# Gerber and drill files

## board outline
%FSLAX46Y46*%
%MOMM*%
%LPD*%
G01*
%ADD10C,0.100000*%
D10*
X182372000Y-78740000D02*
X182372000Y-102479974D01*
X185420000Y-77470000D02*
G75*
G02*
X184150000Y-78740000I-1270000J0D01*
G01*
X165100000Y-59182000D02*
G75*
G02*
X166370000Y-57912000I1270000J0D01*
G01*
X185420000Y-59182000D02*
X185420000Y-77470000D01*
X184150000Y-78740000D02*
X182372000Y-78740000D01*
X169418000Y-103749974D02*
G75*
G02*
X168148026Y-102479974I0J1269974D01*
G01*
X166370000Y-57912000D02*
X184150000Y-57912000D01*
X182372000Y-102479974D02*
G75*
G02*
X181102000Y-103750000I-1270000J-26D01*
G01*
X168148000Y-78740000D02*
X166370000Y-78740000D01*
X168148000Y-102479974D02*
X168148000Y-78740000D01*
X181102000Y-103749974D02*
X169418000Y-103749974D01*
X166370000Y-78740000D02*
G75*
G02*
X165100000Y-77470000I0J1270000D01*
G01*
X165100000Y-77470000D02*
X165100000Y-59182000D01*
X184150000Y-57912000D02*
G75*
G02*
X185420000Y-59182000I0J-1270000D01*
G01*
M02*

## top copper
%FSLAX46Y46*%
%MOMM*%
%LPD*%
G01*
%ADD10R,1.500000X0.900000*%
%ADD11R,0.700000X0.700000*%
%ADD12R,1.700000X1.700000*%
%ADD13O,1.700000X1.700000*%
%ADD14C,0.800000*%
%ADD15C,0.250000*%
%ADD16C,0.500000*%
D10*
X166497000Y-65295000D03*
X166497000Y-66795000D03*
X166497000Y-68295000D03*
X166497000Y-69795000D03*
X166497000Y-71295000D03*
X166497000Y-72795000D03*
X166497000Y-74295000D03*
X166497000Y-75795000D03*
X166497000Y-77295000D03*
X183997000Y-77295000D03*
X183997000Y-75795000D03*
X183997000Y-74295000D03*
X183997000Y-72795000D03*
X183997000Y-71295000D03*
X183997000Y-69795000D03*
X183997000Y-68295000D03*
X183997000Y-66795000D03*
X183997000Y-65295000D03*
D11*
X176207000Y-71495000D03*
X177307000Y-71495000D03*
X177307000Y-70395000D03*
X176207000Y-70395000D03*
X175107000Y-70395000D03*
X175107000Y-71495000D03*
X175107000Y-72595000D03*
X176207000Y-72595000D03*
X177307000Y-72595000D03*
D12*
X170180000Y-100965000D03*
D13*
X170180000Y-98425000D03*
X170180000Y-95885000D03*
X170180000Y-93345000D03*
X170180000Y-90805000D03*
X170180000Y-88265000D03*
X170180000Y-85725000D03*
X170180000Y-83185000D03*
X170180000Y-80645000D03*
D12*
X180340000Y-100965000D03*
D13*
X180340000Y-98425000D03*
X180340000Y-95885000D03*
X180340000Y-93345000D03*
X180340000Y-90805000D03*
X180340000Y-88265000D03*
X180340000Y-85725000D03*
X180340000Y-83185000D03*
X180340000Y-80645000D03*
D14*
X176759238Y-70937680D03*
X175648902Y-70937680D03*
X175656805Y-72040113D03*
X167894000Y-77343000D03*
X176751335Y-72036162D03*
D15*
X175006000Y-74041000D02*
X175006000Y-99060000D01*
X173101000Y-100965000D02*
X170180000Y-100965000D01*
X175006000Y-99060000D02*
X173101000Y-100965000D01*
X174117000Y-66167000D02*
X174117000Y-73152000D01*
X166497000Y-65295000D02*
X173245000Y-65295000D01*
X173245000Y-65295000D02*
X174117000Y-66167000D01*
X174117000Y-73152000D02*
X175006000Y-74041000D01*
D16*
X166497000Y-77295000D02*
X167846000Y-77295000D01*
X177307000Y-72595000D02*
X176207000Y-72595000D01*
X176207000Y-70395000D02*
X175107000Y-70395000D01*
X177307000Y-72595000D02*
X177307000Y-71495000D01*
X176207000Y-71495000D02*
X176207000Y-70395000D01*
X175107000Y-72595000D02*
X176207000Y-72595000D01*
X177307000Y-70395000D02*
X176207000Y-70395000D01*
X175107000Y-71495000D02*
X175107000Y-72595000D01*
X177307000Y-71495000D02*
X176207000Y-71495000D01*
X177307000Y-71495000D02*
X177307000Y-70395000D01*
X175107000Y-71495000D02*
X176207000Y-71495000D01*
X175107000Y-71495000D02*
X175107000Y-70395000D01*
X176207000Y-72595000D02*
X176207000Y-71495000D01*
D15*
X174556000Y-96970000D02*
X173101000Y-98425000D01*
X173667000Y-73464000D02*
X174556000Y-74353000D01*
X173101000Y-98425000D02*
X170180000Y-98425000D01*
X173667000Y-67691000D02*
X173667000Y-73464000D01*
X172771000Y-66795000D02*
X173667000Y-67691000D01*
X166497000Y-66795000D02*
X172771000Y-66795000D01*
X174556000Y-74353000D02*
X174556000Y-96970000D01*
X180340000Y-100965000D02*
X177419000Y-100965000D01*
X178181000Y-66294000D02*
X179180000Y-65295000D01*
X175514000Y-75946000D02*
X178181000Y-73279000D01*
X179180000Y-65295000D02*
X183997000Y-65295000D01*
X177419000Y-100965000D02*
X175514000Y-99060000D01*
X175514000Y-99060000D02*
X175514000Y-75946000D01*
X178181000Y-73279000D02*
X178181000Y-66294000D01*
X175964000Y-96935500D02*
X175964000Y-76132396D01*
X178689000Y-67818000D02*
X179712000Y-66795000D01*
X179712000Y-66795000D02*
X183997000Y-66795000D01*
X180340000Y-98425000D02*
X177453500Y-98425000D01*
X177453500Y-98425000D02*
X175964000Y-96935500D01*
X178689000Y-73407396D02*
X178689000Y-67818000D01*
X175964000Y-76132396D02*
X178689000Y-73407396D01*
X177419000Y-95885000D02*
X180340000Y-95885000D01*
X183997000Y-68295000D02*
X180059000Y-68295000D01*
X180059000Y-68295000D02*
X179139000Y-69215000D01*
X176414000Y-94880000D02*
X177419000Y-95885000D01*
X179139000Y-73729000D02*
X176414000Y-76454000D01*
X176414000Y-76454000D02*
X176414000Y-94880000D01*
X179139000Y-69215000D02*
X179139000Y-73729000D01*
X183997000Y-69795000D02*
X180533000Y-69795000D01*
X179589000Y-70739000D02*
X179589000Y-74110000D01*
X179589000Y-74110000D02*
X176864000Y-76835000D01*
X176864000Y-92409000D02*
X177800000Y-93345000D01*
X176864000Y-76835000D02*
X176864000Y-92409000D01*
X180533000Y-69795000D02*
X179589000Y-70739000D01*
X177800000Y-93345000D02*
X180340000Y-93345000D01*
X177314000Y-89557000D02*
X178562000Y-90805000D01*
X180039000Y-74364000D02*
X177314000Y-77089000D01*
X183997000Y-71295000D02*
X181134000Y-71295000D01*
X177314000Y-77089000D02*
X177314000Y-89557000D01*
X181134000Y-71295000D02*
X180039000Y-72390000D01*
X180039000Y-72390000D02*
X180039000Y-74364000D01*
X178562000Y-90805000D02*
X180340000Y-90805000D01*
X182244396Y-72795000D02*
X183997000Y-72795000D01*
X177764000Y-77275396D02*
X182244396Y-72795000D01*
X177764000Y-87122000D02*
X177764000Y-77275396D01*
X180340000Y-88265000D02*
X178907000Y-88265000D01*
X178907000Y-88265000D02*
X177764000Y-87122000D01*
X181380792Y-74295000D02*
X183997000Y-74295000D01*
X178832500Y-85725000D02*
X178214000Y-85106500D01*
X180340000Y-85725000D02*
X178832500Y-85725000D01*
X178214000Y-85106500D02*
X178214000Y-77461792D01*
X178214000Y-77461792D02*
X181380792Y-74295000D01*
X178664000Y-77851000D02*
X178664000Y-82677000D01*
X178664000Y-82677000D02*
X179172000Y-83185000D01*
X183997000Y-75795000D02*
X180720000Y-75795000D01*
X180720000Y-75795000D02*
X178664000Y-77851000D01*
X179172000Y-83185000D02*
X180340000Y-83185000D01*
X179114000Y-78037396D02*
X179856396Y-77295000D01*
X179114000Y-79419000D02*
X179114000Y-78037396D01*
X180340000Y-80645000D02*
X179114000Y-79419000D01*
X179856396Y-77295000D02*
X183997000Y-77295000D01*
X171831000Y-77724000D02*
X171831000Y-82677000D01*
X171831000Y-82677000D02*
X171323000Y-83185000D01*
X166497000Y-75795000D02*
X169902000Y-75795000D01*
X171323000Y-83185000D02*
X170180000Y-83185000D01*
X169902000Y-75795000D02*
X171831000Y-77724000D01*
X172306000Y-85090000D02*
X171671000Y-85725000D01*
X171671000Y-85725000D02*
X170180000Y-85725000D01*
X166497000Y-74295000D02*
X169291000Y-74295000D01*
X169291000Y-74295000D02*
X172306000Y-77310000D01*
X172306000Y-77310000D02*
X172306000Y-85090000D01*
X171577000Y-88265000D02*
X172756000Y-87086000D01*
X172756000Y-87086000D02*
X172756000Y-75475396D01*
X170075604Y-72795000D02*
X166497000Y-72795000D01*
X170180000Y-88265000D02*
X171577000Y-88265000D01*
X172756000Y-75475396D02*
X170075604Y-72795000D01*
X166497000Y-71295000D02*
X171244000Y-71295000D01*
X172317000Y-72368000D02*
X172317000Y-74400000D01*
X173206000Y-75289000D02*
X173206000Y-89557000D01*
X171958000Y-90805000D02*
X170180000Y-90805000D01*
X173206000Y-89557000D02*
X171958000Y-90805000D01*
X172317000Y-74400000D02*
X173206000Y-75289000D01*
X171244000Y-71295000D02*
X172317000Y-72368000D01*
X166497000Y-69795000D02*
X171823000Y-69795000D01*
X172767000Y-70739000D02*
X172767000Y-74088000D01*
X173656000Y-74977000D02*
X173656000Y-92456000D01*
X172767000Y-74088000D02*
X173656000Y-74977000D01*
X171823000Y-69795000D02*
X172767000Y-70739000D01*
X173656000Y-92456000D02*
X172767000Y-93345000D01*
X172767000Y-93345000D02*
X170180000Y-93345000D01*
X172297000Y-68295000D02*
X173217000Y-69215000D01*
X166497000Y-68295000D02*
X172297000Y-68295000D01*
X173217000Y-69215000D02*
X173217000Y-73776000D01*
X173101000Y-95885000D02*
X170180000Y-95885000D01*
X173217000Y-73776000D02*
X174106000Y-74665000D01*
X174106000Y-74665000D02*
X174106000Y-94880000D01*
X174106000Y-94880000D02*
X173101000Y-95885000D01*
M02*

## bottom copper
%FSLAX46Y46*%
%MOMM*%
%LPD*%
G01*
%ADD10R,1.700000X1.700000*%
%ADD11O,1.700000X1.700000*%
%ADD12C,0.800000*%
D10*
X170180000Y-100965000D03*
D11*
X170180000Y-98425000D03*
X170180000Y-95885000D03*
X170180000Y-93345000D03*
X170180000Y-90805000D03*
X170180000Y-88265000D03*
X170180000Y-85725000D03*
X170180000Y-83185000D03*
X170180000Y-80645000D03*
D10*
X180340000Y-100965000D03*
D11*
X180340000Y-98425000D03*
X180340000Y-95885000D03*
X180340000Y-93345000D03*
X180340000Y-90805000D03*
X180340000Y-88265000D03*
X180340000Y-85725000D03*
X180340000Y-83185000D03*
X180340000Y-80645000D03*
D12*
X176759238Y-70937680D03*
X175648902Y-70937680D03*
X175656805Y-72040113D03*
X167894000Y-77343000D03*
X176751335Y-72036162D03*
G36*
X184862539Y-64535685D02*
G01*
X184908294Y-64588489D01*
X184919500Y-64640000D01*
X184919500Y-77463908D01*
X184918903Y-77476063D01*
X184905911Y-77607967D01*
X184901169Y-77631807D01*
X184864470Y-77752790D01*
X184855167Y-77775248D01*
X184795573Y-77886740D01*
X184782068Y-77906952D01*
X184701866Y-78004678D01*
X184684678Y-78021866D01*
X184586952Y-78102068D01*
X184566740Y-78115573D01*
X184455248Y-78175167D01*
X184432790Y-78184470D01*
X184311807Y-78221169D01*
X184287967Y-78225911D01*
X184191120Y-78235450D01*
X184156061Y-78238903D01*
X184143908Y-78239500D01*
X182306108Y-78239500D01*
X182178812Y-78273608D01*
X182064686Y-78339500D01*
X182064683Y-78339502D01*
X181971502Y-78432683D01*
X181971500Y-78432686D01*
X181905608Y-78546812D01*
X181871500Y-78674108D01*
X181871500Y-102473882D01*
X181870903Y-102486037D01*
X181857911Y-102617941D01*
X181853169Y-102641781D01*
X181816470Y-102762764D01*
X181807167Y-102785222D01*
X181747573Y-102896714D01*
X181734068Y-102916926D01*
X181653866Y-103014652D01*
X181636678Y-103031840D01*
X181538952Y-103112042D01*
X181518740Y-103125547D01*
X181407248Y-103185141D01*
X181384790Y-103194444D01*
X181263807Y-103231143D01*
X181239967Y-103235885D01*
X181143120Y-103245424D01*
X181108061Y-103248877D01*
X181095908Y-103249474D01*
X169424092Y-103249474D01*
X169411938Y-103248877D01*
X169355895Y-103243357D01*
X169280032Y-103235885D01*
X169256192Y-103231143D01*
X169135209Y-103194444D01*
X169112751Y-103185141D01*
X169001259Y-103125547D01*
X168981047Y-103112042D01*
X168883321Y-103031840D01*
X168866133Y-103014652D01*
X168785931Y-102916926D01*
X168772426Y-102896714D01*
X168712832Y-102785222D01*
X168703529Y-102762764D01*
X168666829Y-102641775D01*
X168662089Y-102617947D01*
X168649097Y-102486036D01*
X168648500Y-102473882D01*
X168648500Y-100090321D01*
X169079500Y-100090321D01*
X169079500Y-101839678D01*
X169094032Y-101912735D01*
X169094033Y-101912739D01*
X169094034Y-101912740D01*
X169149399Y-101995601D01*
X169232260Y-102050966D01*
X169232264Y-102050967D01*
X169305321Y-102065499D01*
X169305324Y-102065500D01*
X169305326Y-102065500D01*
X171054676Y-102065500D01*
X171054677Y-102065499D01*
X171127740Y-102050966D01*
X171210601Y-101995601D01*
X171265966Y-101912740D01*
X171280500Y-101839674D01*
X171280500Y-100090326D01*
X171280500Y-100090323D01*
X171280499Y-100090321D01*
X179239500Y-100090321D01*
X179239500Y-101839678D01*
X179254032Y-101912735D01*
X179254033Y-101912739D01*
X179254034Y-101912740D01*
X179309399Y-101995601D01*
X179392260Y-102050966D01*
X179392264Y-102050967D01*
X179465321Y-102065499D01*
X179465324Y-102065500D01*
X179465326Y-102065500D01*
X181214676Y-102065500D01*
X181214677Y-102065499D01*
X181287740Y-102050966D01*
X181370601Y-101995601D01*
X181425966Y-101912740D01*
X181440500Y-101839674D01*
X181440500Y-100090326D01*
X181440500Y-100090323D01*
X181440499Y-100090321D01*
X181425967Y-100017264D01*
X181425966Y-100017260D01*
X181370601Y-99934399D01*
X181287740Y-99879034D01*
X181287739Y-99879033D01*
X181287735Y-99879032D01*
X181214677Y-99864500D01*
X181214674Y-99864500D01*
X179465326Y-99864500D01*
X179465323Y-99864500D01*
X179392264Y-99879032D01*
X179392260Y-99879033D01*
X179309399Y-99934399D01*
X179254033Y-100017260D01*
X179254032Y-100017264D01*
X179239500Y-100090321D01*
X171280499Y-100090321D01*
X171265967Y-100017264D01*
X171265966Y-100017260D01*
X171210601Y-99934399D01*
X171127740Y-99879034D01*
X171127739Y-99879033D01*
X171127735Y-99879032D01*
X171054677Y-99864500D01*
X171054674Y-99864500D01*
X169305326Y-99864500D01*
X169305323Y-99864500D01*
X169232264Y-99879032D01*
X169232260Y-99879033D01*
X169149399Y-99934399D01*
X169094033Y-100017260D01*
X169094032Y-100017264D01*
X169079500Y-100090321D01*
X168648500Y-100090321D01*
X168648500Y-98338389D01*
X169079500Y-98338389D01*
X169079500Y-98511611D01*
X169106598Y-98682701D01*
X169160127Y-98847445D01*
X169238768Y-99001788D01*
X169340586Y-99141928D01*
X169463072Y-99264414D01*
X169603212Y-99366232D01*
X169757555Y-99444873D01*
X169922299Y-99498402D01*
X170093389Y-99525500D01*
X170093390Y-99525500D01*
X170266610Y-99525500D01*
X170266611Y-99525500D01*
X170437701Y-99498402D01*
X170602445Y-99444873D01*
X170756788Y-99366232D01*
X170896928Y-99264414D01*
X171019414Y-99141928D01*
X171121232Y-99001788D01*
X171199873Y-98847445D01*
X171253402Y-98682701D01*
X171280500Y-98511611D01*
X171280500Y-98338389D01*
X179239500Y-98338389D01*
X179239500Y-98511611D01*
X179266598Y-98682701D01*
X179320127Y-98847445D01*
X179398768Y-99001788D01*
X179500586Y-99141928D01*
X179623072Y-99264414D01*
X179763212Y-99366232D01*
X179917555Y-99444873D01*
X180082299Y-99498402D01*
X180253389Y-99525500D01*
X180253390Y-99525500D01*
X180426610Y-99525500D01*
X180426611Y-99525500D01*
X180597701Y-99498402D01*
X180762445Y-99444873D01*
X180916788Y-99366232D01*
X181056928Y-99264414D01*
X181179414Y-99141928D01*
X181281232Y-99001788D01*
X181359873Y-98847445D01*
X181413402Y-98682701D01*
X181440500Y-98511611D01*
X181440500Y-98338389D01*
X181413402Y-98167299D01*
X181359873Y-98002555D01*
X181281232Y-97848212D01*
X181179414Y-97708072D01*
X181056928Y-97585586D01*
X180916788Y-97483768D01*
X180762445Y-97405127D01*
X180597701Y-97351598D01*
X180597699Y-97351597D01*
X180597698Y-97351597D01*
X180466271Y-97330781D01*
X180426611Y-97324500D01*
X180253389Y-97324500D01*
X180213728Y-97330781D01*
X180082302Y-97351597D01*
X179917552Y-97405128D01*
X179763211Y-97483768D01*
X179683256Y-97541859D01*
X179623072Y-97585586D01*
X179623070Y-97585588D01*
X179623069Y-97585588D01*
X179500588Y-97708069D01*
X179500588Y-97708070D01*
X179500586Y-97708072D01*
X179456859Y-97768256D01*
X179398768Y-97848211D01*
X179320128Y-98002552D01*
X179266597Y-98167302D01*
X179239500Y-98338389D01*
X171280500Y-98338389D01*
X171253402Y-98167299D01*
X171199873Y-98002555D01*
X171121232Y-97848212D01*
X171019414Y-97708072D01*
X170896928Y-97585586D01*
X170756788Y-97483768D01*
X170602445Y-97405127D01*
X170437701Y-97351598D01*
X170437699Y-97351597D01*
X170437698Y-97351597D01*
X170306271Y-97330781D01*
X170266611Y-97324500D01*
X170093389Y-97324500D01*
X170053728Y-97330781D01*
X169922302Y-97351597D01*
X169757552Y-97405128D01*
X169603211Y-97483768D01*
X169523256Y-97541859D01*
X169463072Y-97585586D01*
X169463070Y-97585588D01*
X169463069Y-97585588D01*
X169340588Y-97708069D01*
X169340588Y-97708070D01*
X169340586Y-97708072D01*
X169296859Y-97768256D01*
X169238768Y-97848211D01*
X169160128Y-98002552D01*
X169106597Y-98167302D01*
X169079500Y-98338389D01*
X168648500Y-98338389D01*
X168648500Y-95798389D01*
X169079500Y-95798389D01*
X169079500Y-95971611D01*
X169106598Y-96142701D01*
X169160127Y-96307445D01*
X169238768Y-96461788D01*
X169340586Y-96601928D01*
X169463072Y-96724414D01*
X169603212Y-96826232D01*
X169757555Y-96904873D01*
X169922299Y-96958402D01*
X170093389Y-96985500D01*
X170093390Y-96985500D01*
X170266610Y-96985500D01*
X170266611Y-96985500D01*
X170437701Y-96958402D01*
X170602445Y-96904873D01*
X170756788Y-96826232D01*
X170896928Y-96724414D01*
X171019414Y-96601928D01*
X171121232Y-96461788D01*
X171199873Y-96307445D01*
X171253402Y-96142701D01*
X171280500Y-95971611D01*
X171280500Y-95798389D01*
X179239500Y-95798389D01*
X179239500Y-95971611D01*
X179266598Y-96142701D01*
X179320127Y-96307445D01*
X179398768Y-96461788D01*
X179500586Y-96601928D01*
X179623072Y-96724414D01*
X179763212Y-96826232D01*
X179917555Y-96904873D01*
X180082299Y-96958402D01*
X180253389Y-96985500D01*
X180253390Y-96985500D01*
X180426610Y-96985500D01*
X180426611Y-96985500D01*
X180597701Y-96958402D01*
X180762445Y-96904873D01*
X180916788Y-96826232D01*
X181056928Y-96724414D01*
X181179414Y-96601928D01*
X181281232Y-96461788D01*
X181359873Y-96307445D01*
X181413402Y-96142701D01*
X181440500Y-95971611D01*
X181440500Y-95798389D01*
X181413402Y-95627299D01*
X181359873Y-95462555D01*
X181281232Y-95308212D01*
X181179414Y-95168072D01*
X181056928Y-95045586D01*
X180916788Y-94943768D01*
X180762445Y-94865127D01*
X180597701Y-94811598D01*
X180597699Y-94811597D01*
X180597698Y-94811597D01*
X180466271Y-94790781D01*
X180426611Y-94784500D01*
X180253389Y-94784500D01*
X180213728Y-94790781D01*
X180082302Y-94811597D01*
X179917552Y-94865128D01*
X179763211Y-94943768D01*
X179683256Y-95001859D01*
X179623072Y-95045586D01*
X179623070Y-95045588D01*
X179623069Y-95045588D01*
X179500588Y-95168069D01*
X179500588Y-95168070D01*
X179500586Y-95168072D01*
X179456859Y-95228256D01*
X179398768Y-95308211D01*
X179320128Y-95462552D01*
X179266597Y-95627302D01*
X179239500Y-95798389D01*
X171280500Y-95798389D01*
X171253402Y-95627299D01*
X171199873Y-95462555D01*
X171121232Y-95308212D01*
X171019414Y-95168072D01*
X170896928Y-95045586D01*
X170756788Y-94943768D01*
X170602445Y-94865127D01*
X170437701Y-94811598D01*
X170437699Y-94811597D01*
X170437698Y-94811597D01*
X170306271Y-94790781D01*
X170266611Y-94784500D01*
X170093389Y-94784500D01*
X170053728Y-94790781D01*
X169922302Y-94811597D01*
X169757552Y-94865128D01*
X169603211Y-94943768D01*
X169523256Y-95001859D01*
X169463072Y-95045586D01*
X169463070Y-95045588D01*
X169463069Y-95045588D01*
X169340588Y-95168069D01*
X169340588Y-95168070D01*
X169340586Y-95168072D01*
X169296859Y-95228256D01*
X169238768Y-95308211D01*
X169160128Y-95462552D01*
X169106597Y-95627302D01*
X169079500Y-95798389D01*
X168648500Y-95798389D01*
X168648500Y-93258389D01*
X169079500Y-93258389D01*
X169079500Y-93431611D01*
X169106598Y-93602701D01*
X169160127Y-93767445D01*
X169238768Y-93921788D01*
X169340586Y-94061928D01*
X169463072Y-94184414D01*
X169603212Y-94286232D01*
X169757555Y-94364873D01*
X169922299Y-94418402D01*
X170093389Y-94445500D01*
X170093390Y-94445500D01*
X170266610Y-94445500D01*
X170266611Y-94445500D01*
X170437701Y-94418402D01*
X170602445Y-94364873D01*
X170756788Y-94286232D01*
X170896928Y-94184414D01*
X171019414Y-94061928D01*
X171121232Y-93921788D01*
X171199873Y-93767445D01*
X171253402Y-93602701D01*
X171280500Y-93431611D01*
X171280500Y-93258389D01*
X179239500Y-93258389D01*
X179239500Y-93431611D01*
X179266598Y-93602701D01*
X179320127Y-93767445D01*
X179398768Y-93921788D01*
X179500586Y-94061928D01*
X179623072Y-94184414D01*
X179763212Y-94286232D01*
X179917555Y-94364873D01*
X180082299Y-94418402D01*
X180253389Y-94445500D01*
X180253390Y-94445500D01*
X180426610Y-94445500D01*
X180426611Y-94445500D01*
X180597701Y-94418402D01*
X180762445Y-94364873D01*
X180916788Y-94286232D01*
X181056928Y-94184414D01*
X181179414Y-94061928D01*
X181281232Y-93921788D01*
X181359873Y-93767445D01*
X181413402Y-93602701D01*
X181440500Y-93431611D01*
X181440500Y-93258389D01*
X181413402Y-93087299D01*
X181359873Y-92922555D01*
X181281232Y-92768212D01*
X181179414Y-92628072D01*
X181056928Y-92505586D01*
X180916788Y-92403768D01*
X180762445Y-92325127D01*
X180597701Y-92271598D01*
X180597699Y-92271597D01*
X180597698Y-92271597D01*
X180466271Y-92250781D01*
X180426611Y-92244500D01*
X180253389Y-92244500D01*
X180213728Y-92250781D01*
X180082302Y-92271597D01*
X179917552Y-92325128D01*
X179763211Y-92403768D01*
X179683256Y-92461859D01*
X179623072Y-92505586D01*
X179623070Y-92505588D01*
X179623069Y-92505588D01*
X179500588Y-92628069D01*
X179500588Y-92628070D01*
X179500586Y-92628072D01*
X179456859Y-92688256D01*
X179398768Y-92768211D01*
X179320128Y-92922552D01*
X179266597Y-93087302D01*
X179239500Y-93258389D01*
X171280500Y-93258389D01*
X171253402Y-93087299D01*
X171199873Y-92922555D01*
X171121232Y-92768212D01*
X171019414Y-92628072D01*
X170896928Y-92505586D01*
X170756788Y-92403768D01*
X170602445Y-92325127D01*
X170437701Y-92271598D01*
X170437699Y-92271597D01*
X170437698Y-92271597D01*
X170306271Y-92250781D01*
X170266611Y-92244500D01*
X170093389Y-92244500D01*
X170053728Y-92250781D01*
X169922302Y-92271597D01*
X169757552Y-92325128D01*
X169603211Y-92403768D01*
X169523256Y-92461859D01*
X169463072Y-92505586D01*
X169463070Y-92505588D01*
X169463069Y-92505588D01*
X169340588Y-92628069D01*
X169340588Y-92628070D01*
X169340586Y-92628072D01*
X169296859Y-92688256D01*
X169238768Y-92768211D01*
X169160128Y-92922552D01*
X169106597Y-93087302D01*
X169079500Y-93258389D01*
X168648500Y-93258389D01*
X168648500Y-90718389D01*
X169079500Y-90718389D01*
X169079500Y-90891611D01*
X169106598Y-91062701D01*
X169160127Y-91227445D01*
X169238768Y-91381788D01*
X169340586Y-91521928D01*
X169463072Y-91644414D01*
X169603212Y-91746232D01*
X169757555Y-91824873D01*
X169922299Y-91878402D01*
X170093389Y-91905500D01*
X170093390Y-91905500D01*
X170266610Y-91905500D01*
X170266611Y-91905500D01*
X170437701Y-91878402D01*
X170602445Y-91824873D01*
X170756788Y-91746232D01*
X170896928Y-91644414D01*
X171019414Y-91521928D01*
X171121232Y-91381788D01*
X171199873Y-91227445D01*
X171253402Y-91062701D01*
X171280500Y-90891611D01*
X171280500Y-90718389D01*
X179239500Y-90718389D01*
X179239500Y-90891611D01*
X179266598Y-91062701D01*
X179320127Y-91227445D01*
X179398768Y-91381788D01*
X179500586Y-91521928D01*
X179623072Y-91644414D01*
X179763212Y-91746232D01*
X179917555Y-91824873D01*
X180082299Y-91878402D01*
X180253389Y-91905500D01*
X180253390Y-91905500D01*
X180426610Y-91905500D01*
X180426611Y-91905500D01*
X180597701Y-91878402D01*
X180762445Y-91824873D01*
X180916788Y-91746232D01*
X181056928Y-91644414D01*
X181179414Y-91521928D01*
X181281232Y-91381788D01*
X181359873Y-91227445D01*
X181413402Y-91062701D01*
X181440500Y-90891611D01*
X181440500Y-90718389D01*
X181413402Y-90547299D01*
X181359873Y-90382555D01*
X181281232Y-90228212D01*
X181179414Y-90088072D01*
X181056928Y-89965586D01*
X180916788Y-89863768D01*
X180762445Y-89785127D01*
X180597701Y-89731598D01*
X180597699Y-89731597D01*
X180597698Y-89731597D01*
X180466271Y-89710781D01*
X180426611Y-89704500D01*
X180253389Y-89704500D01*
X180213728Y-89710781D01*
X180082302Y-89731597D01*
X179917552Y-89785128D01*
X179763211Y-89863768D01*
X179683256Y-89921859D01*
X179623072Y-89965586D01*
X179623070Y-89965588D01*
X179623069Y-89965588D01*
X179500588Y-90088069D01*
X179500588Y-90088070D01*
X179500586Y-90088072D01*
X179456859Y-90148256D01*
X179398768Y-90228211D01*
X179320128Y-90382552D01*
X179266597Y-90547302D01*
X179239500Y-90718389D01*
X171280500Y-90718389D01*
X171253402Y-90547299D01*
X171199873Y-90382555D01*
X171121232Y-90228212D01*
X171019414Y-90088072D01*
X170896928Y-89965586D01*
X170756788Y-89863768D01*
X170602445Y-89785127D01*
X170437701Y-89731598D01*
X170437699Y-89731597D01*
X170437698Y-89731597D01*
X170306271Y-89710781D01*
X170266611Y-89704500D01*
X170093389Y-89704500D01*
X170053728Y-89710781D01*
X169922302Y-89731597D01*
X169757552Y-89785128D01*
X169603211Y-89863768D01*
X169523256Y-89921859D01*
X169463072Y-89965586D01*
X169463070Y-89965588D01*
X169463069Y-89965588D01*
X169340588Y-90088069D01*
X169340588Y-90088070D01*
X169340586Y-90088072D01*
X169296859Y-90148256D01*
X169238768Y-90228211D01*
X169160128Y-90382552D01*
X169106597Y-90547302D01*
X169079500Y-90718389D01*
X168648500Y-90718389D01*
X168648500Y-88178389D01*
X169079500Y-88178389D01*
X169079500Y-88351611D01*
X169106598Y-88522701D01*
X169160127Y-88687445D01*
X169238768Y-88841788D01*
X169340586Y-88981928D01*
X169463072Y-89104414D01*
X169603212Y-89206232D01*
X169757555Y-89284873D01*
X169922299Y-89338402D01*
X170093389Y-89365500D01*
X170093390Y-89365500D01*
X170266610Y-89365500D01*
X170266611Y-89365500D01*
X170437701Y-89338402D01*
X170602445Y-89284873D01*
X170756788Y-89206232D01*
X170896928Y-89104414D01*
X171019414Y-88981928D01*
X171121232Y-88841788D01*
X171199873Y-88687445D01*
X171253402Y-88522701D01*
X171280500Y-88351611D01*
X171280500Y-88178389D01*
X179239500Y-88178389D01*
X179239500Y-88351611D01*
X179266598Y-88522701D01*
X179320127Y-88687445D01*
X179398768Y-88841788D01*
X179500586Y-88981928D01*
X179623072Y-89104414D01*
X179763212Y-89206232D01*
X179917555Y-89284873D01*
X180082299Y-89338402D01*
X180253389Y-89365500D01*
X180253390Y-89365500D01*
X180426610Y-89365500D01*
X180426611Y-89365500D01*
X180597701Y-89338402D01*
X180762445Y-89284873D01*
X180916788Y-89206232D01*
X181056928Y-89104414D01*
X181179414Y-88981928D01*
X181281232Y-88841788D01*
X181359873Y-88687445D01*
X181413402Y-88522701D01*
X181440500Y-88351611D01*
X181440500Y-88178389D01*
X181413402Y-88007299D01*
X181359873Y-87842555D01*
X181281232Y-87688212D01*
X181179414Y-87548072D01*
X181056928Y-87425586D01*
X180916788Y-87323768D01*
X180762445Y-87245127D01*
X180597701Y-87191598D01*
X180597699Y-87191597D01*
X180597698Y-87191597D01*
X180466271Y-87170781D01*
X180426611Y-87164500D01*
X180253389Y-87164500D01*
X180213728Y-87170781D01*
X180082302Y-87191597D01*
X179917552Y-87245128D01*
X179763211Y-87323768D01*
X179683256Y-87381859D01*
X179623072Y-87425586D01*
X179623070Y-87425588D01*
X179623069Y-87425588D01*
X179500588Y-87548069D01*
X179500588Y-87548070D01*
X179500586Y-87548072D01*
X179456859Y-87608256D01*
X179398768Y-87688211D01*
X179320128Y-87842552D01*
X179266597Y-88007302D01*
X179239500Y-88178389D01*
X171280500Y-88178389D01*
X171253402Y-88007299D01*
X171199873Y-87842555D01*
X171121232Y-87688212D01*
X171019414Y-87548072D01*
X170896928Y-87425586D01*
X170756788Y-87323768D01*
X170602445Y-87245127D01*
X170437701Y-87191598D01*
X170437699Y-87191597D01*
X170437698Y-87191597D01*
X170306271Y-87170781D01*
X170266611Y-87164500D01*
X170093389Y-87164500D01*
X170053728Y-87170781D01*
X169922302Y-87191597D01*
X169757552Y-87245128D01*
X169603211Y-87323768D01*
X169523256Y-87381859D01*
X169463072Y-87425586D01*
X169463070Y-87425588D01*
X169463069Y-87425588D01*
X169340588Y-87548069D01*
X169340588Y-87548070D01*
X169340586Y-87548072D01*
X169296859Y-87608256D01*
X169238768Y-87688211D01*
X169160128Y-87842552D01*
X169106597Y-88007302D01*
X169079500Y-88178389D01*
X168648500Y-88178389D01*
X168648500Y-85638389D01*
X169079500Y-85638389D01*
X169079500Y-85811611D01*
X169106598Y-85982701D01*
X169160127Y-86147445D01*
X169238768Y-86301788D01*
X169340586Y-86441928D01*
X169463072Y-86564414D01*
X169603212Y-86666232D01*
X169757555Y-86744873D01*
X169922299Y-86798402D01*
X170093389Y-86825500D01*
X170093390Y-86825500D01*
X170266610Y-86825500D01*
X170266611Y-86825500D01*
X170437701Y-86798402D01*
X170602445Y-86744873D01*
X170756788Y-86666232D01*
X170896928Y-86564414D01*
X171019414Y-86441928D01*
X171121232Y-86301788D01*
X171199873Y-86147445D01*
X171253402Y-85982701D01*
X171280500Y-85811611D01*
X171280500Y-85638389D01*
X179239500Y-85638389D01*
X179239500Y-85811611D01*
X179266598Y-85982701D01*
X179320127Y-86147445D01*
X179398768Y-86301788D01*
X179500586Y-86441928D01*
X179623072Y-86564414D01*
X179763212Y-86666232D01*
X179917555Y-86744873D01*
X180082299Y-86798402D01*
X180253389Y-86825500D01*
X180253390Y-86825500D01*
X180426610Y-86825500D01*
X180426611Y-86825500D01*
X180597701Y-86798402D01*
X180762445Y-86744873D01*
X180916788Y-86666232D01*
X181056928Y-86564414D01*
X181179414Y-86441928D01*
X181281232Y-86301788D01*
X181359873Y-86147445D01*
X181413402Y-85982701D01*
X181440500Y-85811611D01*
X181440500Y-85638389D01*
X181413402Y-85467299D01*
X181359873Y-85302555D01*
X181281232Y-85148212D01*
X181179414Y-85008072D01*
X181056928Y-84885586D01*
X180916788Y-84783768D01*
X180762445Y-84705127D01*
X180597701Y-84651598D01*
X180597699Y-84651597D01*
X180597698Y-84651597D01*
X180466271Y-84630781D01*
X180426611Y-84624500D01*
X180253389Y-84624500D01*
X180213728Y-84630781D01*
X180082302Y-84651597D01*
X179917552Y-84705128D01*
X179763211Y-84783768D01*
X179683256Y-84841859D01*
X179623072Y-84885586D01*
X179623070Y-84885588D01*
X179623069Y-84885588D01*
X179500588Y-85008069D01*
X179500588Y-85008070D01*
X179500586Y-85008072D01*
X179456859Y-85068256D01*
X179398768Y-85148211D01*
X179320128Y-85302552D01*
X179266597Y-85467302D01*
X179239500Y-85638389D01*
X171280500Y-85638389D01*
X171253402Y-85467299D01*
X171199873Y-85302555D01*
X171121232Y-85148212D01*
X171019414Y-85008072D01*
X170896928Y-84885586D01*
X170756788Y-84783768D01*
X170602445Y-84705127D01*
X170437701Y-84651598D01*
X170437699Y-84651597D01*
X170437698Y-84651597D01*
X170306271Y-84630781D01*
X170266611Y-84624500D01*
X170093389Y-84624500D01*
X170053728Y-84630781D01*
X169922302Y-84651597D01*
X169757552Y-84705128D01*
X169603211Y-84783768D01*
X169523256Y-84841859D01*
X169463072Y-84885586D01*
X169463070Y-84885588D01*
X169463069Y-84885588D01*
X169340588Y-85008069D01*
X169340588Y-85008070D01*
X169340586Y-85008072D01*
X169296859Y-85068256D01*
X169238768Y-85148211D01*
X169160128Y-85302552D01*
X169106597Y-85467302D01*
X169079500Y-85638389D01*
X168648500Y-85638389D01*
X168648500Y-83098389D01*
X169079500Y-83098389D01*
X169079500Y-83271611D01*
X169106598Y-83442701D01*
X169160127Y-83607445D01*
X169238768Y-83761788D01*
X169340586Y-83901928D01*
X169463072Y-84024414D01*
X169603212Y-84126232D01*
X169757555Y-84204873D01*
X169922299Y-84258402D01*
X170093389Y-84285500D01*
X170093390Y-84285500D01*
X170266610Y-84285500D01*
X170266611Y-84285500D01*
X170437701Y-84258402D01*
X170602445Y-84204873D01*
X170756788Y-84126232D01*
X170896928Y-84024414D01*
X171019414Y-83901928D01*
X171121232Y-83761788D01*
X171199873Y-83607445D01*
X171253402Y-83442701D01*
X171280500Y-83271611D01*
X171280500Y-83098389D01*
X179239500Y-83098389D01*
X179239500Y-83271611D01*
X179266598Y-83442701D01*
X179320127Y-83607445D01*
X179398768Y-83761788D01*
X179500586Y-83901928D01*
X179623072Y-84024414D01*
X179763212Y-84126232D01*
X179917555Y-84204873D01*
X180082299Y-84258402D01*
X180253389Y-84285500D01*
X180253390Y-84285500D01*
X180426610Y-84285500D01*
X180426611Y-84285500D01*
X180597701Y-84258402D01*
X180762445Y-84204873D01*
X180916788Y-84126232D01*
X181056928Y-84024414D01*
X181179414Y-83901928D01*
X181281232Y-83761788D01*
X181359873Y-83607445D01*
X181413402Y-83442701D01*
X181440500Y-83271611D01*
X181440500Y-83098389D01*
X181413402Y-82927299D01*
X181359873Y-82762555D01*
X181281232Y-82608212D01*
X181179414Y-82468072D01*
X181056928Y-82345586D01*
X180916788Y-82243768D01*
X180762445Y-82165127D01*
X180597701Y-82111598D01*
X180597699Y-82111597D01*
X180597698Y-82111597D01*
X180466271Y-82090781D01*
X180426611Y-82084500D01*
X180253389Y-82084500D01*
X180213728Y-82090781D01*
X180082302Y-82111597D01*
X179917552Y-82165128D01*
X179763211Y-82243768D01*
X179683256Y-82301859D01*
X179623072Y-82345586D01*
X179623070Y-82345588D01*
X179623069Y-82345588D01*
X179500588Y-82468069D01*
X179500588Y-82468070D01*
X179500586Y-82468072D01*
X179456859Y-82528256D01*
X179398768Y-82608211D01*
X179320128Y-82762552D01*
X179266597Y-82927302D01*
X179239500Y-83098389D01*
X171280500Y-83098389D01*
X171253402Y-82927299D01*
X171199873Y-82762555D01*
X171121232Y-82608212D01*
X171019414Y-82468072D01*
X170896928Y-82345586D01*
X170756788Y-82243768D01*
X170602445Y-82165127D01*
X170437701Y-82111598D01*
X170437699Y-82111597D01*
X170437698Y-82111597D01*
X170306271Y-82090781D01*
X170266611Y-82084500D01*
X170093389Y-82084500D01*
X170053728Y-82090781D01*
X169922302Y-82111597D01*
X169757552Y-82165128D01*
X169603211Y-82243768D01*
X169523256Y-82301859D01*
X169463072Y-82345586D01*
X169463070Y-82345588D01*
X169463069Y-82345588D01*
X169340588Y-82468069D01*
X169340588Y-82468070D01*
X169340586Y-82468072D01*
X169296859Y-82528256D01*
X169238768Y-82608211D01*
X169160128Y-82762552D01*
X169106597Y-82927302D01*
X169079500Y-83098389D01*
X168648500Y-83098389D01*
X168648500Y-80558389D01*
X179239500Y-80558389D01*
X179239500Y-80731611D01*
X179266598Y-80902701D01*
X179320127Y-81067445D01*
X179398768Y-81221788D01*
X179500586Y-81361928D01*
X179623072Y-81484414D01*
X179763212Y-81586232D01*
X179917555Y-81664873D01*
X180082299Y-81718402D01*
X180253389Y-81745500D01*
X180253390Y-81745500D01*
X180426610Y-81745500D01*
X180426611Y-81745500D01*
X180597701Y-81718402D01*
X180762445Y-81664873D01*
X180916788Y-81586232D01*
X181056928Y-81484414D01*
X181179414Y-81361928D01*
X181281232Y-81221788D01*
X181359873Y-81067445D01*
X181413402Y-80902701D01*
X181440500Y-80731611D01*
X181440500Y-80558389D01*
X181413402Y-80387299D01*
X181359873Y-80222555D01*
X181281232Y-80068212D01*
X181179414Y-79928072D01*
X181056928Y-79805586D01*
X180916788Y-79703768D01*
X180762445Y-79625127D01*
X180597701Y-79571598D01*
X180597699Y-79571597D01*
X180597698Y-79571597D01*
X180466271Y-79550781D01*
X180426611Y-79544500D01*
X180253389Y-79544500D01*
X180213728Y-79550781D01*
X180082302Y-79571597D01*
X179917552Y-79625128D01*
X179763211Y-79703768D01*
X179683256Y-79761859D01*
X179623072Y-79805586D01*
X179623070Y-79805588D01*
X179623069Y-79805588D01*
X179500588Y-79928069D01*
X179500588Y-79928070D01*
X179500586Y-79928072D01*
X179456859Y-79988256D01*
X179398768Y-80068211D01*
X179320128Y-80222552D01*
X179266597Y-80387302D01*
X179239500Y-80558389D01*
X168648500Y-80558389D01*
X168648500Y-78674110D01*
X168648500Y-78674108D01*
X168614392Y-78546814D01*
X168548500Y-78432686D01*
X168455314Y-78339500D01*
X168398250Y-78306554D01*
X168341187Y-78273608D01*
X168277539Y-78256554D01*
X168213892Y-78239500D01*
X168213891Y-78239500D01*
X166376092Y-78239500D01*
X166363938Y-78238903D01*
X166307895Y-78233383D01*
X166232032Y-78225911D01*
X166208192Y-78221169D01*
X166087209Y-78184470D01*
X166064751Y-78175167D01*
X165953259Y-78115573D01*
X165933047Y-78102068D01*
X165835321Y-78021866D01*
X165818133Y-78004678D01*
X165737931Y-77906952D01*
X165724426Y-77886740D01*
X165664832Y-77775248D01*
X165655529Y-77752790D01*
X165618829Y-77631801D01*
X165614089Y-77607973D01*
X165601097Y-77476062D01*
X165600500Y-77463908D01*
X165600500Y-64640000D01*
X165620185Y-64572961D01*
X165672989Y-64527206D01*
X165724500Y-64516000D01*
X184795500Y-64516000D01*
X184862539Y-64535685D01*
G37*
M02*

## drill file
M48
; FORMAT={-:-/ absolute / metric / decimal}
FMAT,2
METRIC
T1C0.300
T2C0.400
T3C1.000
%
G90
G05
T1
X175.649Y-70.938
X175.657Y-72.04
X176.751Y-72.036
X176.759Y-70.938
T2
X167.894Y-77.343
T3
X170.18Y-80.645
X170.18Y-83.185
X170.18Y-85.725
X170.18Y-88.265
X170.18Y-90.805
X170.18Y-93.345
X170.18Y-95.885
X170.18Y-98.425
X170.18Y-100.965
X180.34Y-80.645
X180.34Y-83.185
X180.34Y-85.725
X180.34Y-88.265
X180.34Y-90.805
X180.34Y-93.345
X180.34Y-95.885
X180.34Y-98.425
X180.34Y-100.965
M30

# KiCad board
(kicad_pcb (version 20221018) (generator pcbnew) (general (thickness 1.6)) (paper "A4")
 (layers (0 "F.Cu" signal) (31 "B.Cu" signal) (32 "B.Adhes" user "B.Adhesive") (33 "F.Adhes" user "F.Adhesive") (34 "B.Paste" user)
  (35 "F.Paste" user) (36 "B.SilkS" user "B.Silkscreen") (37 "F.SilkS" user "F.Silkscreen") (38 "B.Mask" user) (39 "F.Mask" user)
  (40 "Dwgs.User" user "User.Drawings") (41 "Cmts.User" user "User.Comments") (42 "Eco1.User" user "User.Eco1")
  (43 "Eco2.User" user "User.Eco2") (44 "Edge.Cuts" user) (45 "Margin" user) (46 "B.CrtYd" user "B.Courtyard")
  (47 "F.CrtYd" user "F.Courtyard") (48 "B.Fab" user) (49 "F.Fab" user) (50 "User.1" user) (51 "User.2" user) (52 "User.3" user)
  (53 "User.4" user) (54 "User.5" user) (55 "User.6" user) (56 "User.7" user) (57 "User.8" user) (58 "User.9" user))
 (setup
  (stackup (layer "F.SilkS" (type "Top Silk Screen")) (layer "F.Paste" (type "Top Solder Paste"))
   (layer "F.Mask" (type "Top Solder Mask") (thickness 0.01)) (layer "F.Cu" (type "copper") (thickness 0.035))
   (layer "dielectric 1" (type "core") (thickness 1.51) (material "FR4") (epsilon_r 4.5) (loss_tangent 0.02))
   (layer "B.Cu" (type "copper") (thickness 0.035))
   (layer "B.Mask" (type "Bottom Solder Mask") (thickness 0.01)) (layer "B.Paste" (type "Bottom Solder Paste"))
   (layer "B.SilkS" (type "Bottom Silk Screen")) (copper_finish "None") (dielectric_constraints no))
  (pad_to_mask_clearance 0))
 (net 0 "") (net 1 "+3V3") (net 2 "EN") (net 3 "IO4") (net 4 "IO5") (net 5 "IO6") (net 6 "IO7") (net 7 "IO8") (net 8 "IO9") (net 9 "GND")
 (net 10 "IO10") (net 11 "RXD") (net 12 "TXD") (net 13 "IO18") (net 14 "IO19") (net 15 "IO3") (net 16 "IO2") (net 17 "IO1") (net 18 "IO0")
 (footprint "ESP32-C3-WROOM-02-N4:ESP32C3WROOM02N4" (layer "F.Cu") (at 176.207 71.495)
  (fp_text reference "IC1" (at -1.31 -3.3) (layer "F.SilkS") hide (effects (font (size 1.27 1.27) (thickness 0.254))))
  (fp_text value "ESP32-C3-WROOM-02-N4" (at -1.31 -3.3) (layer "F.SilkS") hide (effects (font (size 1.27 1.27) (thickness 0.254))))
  (pad "1" smd rect (at -9.71 -6.2 90) (size 0.9 1.5) (layers "F.Cu" "F.Paste" "F.Mask") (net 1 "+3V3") (thermal_bridge_angle 45))
  (pad "2" smd rect (at -9.71 -4.7 90) (size 0.9 1.5) (layers "F.Cu" "F.Paste" "F.Mask") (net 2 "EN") (thermal_bridge_angle 45))
  (pad "3" smd rect (at -9.71 -3.2 90) (size 0.9 1.5) (layers "F.Cu" "F.Paste" "F.Mask") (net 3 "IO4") (thermal_bridge_angle 45))
  (pad "4" smd rect (at -9.71 -1.7 90) (size 0.9 1.5) (layers "F.Cu" "F.Paste" "F.Mask") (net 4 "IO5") (thermal_bridge_angle 45))
  (pad "5" smd rect (at -9.71 -0.2 90) (size 0.9 1.5) (layers "F.Cu" "F.Paste" "F.Mask") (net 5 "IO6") (thermal_bridge_angle 45))
  (pad "6" smd rect (at -9.71 1.3 90) (size 0.9 1.5) (layers "F.Cu" "F.Paste" "F.Mask") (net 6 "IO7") (thermal_bridge_angle 45))
  (pad "7" smd rect (at -9.71 2.8 90) (size 0.9 1.5) (layers "F.Cu" "F.Paste" "F.Mask") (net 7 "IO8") (thermal_bridge_angle 45))
  (pad "8" smd rect (at -9.71 4.3 90) (size 0.9 1.5) (layers "F.Cu" "F.Paste" "F.Mask") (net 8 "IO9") (thermal_bridge_angle 45))
  (pad "9" smd rect (at -9.71 5.8 90) (size 0.9 1.5) (layers "F.Cu" "F.Paste" "F.Mask") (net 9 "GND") (thermal_bridge_angle 45))
  (pad "10" smd rect (at 7.79 5.8 90) (size 0.9 1.5) (layers "F.Cu" "F.Paste" "F.Mask") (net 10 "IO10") (thermal_bridge_angle 45))
  (pad "11" smd rect (at 7.79 4.3 90) (size 0.9 1.5) (layers "F.Cu" "F.Paste" "F.Mask") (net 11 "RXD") (thermal_bridge_angle 45))
  (pad "12" smd rect (at 7.79 2.8 90) (size 0.9 1.5) (layers "F.Cu" "F.Paste" "F.Mask") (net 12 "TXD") (thermal_bridge_angle 45))
  (pad "13" smd rect (at 7.79 1.3 90) (size 0.9 1.5) (layers "F.Cu" "F.Paste" "F.Mask") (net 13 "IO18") (thermal_bridge_angle 45))
  (pad "14" smd rect (at 7.79 -0.2 90) (size 0.9 1.5) (layers "F.Cu" "F.Paste" "F.Mask") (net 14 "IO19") (thermal_bridge_angle 45))
  (pad "15" smd rect (at 7.79 -1.7 90) (size 0.9 1.5) (layers "F.Cu" "F.Paste" "F.Mask") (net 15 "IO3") (thermal_bridge_angle 45))
  (pad "16" smd rect (at 7.79 -3.2 90) (size 0.9 1.5) (layers "F.Cu" "F.Paste" "F.Mask") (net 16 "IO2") (thermal_bridge_angle 45))
  (pad "17" smd rect (at 7.79 -4.7 90) (size 0.9 1.5) (layers "F.Cu" "F.Paste" "F.Mask") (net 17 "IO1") (thermal_bridge_angle 45))
  (pad "18" smd rect (at 7.79 -6.2 90) (size 0.9 1.5) (layers "F.Cu" "F.Paste" "F.Mask") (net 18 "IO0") (thermal_bridge_angle 45))
  (pad "19" smd rect (at 0 0 90) (size 0.7 0.7) (layers "F.Cu" "F.Paste" "F.Mask") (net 9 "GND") (thermal_bridge_angle 45))
  (pad "20" smd rect (at 1.1 0 90) (size 0.7 0.7) (layers "F.Cu" "F.Paste" "F.Mask") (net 9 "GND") (thermal_bridge_angle 45))
  (pad "21" smd rect (at 1.1 -1.1 90) (size 0.7 0.7) (layers "F.Cu" "F.Paste" "F.Mask") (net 9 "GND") (thermal_bridge_angle 45))
  (pad "22" smd rect (at 0 -1.1 90) (size 0.7 0.7) (layers "F.Cu" "F.Paste" "F.Mask") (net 9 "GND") (thermal_bridge_angle 45))
  (pad "23" smd rect (at -1.1 -1.1 90) (size 0.7 0.7) (layers "F.Cu" "F.Paste" "F.Mask") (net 9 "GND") (thermal_bridge_angle 45))
  (pad "24" smd rect (at -1.1 0 90) (size 0.7 0.7) (layers "F.Cu" "F.Paste" "F.Mask") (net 9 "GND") (thermal_bridge_angle 45))
  (pad "25" smd rect (at -1.1 1.1 90) (size 0.7 0.7) (layers "F.Cu" "F.Paste" "F.Mask") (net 9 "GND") (thermal_bridge_angle 45))
  (pad "26" smd rect (at 0 1.1 90) (size 0.7 0.7) (layers "F.Cu" "F.Paste" "F.Mask") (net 9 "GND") (thermal_bridge_angle 45))
  (pad "27" smd rect (at 1.1 1.1 90) (size 0.7 0.7) (layers "F.Cu" "F.Paste" "F.Mask") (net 9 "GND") (thermal_bridge_angle 45)))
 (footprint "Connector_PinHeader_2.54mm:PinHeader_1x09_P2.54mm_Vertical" (layer "B.Cu") (at 170.18 100.965)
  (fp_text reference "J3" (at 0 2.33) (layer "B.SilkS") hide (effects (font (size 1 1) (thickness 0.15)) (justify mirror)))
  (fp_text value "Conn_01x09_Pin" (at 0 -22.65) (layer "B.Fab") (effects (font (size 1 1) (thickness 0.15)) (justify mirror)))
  (pad "1" thru_hole rect (at 0 0) (size 1.7 1.7) (drill 1) (layers "*.Cu" "*.Mask") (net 1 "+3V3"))
  (pad "2" thru_hole oval (at 0 -2.54) (size 1.7 1.7) (drill 1) (layers "*.Cu" "*.Mask") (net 2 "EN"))
  (pad "3" thru_hole oval (at 0 -5.08) (size 1.7 1.7) (drill 1) (layers "*.Cu" "*.Mask") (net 3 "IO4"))
  (pad "4" thru_hole oval (at 0 -7.62) (size 1.7 1.7) (drill 1) (layers "*.Cu" "*.Mask") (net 4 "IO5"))
  (pad "5" thru_hole oval (at 0 -10.16) (size 1.7 1.7) (drill 1) (layers "*.Cu" "*.Mask") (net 5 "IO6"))
  (pad "6" thru_hole oval (at 0 -12.7) (size 1.7 1.7) (drill 1) (layers "*.Cu" "*.Mask") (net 6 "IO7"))
  (pad "7" thru_hole oval (at 0 -15.24) (size 1.7 1.7) (drill 1) (layers "*.Cu" "*.Mask") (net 7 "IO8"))
  (pad "8" thru_hole oval (at 0 -17.78) (size 1.7 1.7) (drill 1) (layers "*.Cu" "*.Mask") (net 8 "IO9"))
  (pad "9" thru_hole oval (at 0 -20.32) (size 1.7 1.7) (drill 1) (layers "*.Cu" "*.Mask") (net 9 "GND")))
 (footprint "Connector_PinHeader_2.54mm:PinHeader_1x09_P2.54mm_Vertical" (layer "B.Cu") (at 180.34 100.965)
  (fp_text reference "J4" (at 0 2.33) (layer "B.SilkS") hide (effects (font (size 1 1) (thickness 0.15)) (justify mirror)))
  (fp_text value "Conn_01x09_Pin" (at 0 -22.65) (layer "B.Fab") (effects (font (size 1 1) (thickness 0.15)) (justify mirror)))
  (pad "1" thru_hole rect (at 0 0) (size 1.7 1.7) (drill 1) (layers "*.Cu" "*.Mask") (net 18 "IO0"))
  (pad "2" thru_hole oval (at 0 -2.54) (size 1.7 1.7) (drill 1) (layers "*.Cu" "*.Mask") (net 17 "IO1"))
  (pad "3" thru_hole oval (at 0 -5.08) (size 1.7 1.7) (drill 1) (layers "*.Cu" "*.Mask") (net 16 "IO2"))
  (pad "4" thru_hole oval (at 0 -7.62) (size 1.7 1.7) (drill 1) (layers "*.Cu" "*.Mask") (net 15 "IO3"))
  (pad "5" thru_hole oval (at 0 -10.16) (size 1.7 1.7) (drill 1) (layers "*.Cu" "*.Mask") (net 14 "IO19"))
  (pad "6" thru_hole oval (at 0 -12.7) (size 1.7 1.7) (drill 1) (layers "*.Cu" "*.Mask") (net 13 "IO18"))
  (pad "7" thru_hole oval (at 0 -15.24) (size 1.7 1.7) (drill 1) (layers "*.Cu" "*.Mask") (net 12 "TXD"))
  (pad "8" thru_hole oval (at 0 -17.78) (size 1.7 1.7) (drill 1) (layers "*.Cu" "*.Mask") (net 11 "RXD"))
  (pad "9" thru_hole oval (at 0 -20.32) (size 1.7 1.7) (drill 1) (layers "*.Cu" "*.Mask") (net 10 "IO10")))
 (gr_line (start 182.372 78.74) (end 182.372 102.479974) (stroke (width 0.1) (type default)) (layer "Edge.Cuts"))
 (gr_arc (start 185.42 77.47) (mid 185.048026 78.368026) (end 184.15 78.74) (stroke (width 0.1) (type default)) (layer "Edge.Cuts"))
 (gr_arc (start 165.1 59.182) (mid 165.471974 58.283974) (end 166.37 57.912) (stroke (width 0.1) (type default)) (layer "Edge.Cuts"))
 (gr_line (start 185.42 59.182) (end 185.42 77.47) (stroke (width 0.1) (type default)) (layer "Edge.Cuts"))
 (gr_line (start 184.15 78.74) (end 182.372 78.74) (stroke (width 0.1) (type default)) (layer "Edge.Cuts"))
 (gr_arc (start 169.418 103.749974) (mid 168.519974 103.378) (end 168.148 102.479974) (stroke (width 0.1) (type default))
  (layer "Edge.Cuts"))
 (gr_line (start 166.37 57.912) (end 184.15 57.912) (stroke (width 0.1) (type default)) (layer "Edge.Cuts"))
 (gr_arc (start 182.372 102.479974) (mid 182.000026 103.378) (end 181.102 103.749974) (stroke (width 0.1) (type default))
  (layer "Edge.Cuts"))
 (gr_line (start 168.148 78.74) (end 166.37 78.74) (stroke (width 0.1) (type default)) (layer "Edge.Cuts"))
 (gr_line (start 168.148 102.479974) (end 168.148 78.74) (stroke (width 0.1) (type default)) (layer "Edge.Cuts"))
 (gr_line (start 181.102 103.749974) (end 169.418 103.749974) (stroke (width 0.1) (type default)) (layer "Edge.Cuts"))
 (gr_arc (start 166.37 78.74) (mid 165.471974 78.368026) (end 165.1 77.47) (stroke (width 0.1) (type default)) (layer "Edge.Cuts"))
 (gr_line (start 165.1 77.47) (end 165.1 59.182) (stroke (width 0.1) (type default)) (layer "Edge.Cuts"))
 (gr_arc (start 184.15 57.912) (mid 185.048026 58.283974) (end 185.42 59.182) (stroke (width 0.1) (type default)) (layer "Edge.Cuts"))
 (segment (start 175.006 74.041) (end 175.006 99.06) (width 0.25) (layer "F.Cu") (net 1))
 (segment (start 173.101 100.965) (end 170.18 100.965) (width 0.25) (layer "F.Cu") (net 1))
 (segment (start 175.006 99.06) (end 173.101 100.965) (width 0.25) (layer "F.Cu") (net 1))
 (segment (start 174.117 66.167) (end 174.117 73.152) (width 0.25) (layer "F.Cu") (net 1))
 (segment (start 166.497 65.295) (end 173.245 65.295) (width 0.25) (layer "F.Cu") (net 1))
 (segment (start 173.245 65.295) (end 174.117 66.167) (width 0.25) (layer "F.Cu") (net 1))
 (segment (start 174.117 73.152) (end 175.006 74.041) (width 0.25) (layer "F.Cu") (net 1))
 (segment (start 166.497 77.295) (end 167.846 77.295) (width 0.5) (layer "F.Cu") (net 9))
 (segment (start 177.307 72.595) (end 176.207 72.595) (width 0.5) (layer "F.Cu") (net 9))
 (segment (start 176.207 70.395) (end 175.107 70.395) (width 0.5) (layer "F.Cu") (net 9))
 (segment (start 177.307 72.595) (end 177.307 71.495) (width 0.5) (layer "F.Cu") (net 9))
 (segment (start 176.207 71.495) (end 176.207 70.395) (width 0.5) (layer "F.Cu") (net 9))
 (segment (start 175.107 72.595) (end 176.207 72.595) (width 0.5) (layer "F.Cu") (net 9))
 (segment (start 177.307 70.395) (end 176.207 70.395) (width 0.5) (layer "F.Cu") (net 9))
 (segment (start 175.107 71.495) (end 175.107 72.595) (width 0.5) (layer "F.Cu") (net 9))
 (segment (start 177.307 71.495) (end 176.207 71.495) (width 0.5) (layer "F.Cu") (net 9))
 (segment (start 177.307 71.495) (end 177.307 70.395) (width 0.5) (layer "F.Cu") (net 9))
 (segment (start 175.107 71.495) (end 176.207 71.495) (width 0.5) (layer "F.Cu") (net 9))
 (segment (start 175.107 71.495) (end 175.107 70.395) (width 0.5) (layer "F.Cu") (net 9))
 (segment (start 176.207 72.595) (end 176.207 71.495) (width 0.5) (layer "F.Cu") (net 9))
 (via (at 176.759238 70.93768) (size 0.8) (drill 0.3) (layers "F.Cu" "B.Cu") (free) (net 9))
 (via (at 175.648902 70.93768) (size 0.8) (drill 0.3) (layers "F.Cu" "B.Cu") (free) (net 9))
 (via (at 175.656805 72.040113) (size 0.8) (drill 0.3) (layers "F.Cu" "B.Cu") (free) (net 9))
 (via (at 167.894 77.343) (size 0.8) (drill 0.4) (layers "F.Cu" "B.Cu") (free) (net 9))
 (via (at 176.751335 72.036162) (size 0.8) (drill 0.3) (layers "F.Cu" "B.Cu") (free) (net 9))
 (segment (start 174.556 96.97) (end 173.101 98.425) (width 0.25) (layer "F.Cu") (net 2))
 (segment (start 173.667 73.464) (end 174.556 74.353) (width 0.25) (layer "F.Cu") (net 2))
 (segment (start 173.101 98.425) (end 170.18 98.425) (width 0.25) (layer "F.Cu") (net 2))
 (segment (start 173.667 67.691) (end 173.667 73.464) (width 0.25) (layer "F.Cu") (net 2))
 (segment (start 172.771 66.795) (end 173.667 67.691) (width 0.25) (layer "F.Cu") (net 2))
 (segment (start 166.497 66.795) (end 172.771 66.795) (width 0.25) (layer "F.Cu") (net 2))
 (segment (start 174.556 74.353) (end 174.556 96.97) (width 0.25) (layer "F.Cu") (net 2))
 (segment (start 180.34 100.965) (end 177.419 100.965) (width 0.25) (layer "F.Cu") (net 18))
 (segment (start 178.181 66.294) (end 179.18 65.295) (width 0.25) (layer "F.Cu") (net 18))
 (segment (start 175.514 75.946) (end 178.181 73.279) (width 0.25) (layer "F.Cu") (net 18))
 (segment (start 179.18 65.295) (end 183.997 65.295) (width 0.25) (layer "F.Cu") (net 18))
 (segment (start 177.419 100.965) (end 175.514 99.06) (width 0.25) (layer "F.Cu") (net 18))
 (segment (start 175.514 99.06) (end 175.514 75.946) (width 0.25) (layer "F.Cu") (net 18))
 (segment (start 178.181 73.279) (end 178.181 66.294) (width 0.25) (layer "F.Cu") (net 18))
 (segment (start 175.964 96.9355) (end 175.964 76.132396) (width 0.25) (layer "F.Cu") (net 17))
 (segment (start 178.689 67.818) (end 179.712 66.795) (width 0.25) (layer "F.Cu") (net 17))
 (segment (start 179.712 66.795) (end 183.997 66.795) (width 0.25) (layer "F.Cu") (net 17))
 (segment (start 180.34 98.425) (end 177.4535 98.425) (width 0.25) (layer "F.Cu") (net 17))
 (segment (start 177.4535 98.425) (end 175.964 96.9355) (width 0.25) (layer "F.Cu") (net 17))
 (segment (start 178.689 73.407396) (end 178.689 67.818) (width 0.25) (layer "F.Cu") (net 17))
 (segment (start 175.964 76.132396) (end 178.689 73.407396) (width 0.25) (layer "F.Cu") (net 17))
 (segment (start 177.419 95.885) (end 180.34 95.885) (width 0.25) (layer "F.Cu") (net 16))
 (segment (start 183.997 68.295) (end 180.059 68.295) (width 0.25) (layer "F.Cu") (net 16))
 (segment (start 180.059 68.295) (end 179.139 69.215) (width 0.25) (layer "F.Cu") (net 16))
 (segment (start 176.414 94.88) (end 177.419 95.885) (width 0.25) (layer "F.Cu") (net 16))
 (segment (start 179.139 73.729) (end 176.414 76.454) (width 0.25) (layer "F.Cu") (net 16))
 (segment (start 176.414 76.454) (end 176.414 94.88) (width 0.25) (layer "F.Cu") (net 16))
 (segment (start 179.139 69.215) (end 179.139 73.729) (width 0.25) (layer "F.Cu") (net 16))
 (segment (start 183.997 69.795) (end 180.533 69.795) (width 0.25) (layer "F.Cu") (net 15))
 (segment (start 179.589 70.739) (end 179.589 74.11) (width 0.25) (layer "F.Cu") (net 15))
 (segment (start 179.589 74.11) (end 176.864 76.835) (width 0.25) (layer "F.Cu") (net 15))
 (segment (start 176.864 92.409) (end 177.8 93.345) (width 0.25) (layer "F.Cu") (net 15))
 (segment (start 176.864 76.835) (end 176.864 92.409) (width 0.25) (layer "F.Cu") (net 15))
 (segment (start 180.533 69.795) (end 179.589 70.739) (width 0.25) (layer "F.Cu") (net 15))
 (segment (start 177.8 93.345) (end 180.34 93.345) (width 0.25) (layer "F.Cu") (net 15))
 (segment (start 177.314 89.557) (end 178.562 90.805) (width 0.25) (layer "F.Cu") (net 14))
 (segment (start 180.039 74.364) (end 177.314 77.089) (width 0.25) (layer "F.Cu") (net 14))
 (segment (start 183.997 71.295) (end 181.134 71.295) (width 0.25) (layer "F.Cu") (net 14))
 (segment (start 177.314 77.089) (end 177.314 89.557) (width 0.25) (layer "F.Cu") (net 14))
 (segment (start 181.134 71.295) (end 180.039 72.39) (width 0.25) (layer "F.Cu") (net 14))
 (segment (start 180.039 72.39) (end 180.039 74.364) (width 0.25) (layer "F.Cu") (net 14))
 (segment (start 178.562 90.805) (end 180.34 90.805) (width 0.25) (layer "F.Cu") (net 14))
 (segment (start 182.244396 72.795) (end 183.997 72.795) (width 0.25) (layer "F.Cu") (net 13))
 (segment (start 177.764 77.275396) (end 182.244396 72.795) (width 0.25) (layer "F.Cu") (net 13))
 (segment (start 177.764 87.122) (end 177.764 77.275396) (width 0.25) (layer "F.Cu") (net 13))
 (segment (start 180.34 88.265) (end 178.907 88.265) (width 0.25) (layer "F.Cu") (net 13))
 (segment (start 178.907 88.265) (end 177.764 87.122) (width 0.25) (layer "F.Cu") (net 13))
 (segment (start 181.380792 74.295) (end 183.997 74.295) (width 0.25) (layer "F.Cu") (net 12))
 (segment (start 178.8325 85.725) (end 178.214 85.1065) (width 0.25) (layer "F.Cu") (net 12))
 (segment (start 180.34 85.725) (end 178.8325 85.725) (width 0.25) (layer "F.Cu") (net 12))
 (segment (start 178.214 85.1065) (end 178.214 77.461792) (width 0.25) (layer "F.Cu") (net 12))
 (segment (start 178.214 77.461792) (end 181.380792 74.295) (width 0.25) (layer "F.Cu") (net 12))
 (segment (start 178.664 77.851) (end 178.664 82.677) (width 0.25) (layer "F.Cu") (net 11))
 (segment (start 178.664 82.677) (end 179.172 83.185) (width 0.25) (layer "F.Cu") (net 11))
 (segment (start 183.997 75.795) (end 180.72 75.795) (width 0.25) (layer "F.Cu") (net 11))
 (segment (start 180.72 75.795) (end 178.664 77.851) (width 0.25) (layer "F.Cu") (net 11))
 (segment (start 179.172 83.185) (end 180.34 83.185) (width 0.25) (layer "F.Cu") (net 11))
 (segment (start 179.114 78.037396) (end 179.856396 77.295) (width 0.25) (layer "F.Cu") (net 10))
 (segment (start 179.114 79.419) (end 179.114 78.037396) (width 0.25) (layer "F.Cu") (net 10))
 (segment (start 180.34 80.645) (end 179.114 79.419) (width 0.25) (layer "F.Cu") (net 10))
 (segment (start 179.856396 77.295) (end 183.997 77.295) (width 0.25) (layer "F.Cu") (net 10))
 (segment (start 171.831 77.724) (end 171.831 82.677) (width 0.25) (layer "F.Cu") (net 8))
 (segment (start 171.831 82.677) (end 171.323 83.185) (width 0.25) (layer "F.Cu") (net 8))
 (segment (start 166.497 75.795) (end 169.902 75.795) (width 0.25) (layer "F.Cu") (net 8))
 (segment (start 171.323 83.185) (end 170.18 83.185) (width 0.25) (layer "F.Cu") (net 8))
 (segment (start 169.902 75.795) (end 171.831 77.724) (width 0.25) (layer "F.Cu") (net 8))
 (segment (start 172.306 85.09) (end 171.671 85.725) (width 0.25) (layer "F.Cu") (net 7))
 (segment (start 171.671 85.725) (end 170.18 85.725) (width 0.25) (layer "F.Cu") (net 7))
 (segment (start 166.497 74.295) (end 169.291 74.295) (width 0.25) (layer "F.Cu") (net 7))
 (segment (start 169.291 74.295) (end 172.306 77.31) (width 0.25) (layer "F.Cu") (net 7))
 (segment (start 172.306 77.31) (end 172.306 85.09) (width 0.25) (layer "F.Cu") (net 7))
 (segment (start 171.577 88.265) (end 172.756 87.086) (width 0.25) (layer "F.Cu") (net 6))
 (segment (start 172.756 87.086) (end 172.756 75.475396) (width 0.25) (layer "F.Cu") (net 6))
 (segment (start 170.075604 72.795) (end 166.497 72.795) (width 0.25) (layer "F.Cu") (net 6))
 (segment (start 170.18 88.265) (end 171.577 88.265) (width 0.25) (layer "F.Cu") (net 6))
 (segment (start 172.756 75.475396) (end 170.075604 72.795) (width 0.25) (layer "F.Cu") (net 6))
 (segment (start 166.497 71.295) (end 171.244 71.295) (width 0.25) (layer "F.Cu") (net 5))
 (segment (start 172.317 72.368) (end 172.317 74.4) (width 0.25) (layer "F.Cu") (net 5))
 (segment (start 173.206 75.289) (end 173.206 89.557) (width 0.25) (layer "F.Cu") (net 5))
 (segment (start 171.958 90.805) (end 170.18 90.805) (width 0.25) (layer "F.Cu") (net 5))
 (segment (start 173.206 89.557) (end 171.958 90.805) (width 0.25) (layer "F.Cu") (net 5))
 (segment (start 172.317 74.4) (end 173.206 75.289) (width 0.25) (layer "F.Cu") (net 5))
 (segment (start 171.244 71.295) (end 172.317 72.368) (width 0.25) (layer "F.Cu") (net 5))
 (segment (start 166.497 69.795) (end 171.823 69.795) (width 0.25) (layer "F.Cu") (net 4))
 (segment (start 172.767 70.739) (end 172.767 74.088) (width 0.25) (layer "F.Cu") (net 4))
 (segment (start 173.656 74.977) (end 173.656 92.456) (width 0.25) (layer "F.Cu") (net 4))
 (segment (start 172.767 74.088) (end 173.656 74.977) (width 0.25) (layer "F.Cu") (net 4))
 (segment (start 171.823 69.795) (end 172.767 70.739) (width 0.25) (layer "F.Cu") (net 4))
 (segment (start 173.656 92.456) (end 172.767 93.345) (width 0.25) (layer "F.Cu") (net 4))
 (segment (start 172.767 93.345) (end 170.18 93.345) (width 0.25) (layer "F.Cu") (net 4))
 (segment (start 172.297 68.295) (end 173.217 69.215) (width 0.25) (layer "F.Cu") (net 3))
 (segment (start 166.497 68.295) (end 172.297 68.295) (width 0.25) (layer "F.Cu") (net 3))
 (segment (start 173.217 69.215) (end 173.217 73.776) (width 0.25) (layer "F.Cu") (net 3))
 (segment (start 173.101 95.885) (end 170.18 95.885) (width 0.25) (layer "F.Cu") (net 3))
 (segment (start 173.217 73.776) (end 174.106 74.665) (width 0.25) (layer "F.Cu") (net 3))
 (segment (start 174.106 74.665) (end 174.106 94.88) (width 0.25) (layer "F.Cu") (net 3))
 (segment (start 174.106 94.88) (end 173.101 95.885) (width 0.25) (layer "F.Cu") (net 3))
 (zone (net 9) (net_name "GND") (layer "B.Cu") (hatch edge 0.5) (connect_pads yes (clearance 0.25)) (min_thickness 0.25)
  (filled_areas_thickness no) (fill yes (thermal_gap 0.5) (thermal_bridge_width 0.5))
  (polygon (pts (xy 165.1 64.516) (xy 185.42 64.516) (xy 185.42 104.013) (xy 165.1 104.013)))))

